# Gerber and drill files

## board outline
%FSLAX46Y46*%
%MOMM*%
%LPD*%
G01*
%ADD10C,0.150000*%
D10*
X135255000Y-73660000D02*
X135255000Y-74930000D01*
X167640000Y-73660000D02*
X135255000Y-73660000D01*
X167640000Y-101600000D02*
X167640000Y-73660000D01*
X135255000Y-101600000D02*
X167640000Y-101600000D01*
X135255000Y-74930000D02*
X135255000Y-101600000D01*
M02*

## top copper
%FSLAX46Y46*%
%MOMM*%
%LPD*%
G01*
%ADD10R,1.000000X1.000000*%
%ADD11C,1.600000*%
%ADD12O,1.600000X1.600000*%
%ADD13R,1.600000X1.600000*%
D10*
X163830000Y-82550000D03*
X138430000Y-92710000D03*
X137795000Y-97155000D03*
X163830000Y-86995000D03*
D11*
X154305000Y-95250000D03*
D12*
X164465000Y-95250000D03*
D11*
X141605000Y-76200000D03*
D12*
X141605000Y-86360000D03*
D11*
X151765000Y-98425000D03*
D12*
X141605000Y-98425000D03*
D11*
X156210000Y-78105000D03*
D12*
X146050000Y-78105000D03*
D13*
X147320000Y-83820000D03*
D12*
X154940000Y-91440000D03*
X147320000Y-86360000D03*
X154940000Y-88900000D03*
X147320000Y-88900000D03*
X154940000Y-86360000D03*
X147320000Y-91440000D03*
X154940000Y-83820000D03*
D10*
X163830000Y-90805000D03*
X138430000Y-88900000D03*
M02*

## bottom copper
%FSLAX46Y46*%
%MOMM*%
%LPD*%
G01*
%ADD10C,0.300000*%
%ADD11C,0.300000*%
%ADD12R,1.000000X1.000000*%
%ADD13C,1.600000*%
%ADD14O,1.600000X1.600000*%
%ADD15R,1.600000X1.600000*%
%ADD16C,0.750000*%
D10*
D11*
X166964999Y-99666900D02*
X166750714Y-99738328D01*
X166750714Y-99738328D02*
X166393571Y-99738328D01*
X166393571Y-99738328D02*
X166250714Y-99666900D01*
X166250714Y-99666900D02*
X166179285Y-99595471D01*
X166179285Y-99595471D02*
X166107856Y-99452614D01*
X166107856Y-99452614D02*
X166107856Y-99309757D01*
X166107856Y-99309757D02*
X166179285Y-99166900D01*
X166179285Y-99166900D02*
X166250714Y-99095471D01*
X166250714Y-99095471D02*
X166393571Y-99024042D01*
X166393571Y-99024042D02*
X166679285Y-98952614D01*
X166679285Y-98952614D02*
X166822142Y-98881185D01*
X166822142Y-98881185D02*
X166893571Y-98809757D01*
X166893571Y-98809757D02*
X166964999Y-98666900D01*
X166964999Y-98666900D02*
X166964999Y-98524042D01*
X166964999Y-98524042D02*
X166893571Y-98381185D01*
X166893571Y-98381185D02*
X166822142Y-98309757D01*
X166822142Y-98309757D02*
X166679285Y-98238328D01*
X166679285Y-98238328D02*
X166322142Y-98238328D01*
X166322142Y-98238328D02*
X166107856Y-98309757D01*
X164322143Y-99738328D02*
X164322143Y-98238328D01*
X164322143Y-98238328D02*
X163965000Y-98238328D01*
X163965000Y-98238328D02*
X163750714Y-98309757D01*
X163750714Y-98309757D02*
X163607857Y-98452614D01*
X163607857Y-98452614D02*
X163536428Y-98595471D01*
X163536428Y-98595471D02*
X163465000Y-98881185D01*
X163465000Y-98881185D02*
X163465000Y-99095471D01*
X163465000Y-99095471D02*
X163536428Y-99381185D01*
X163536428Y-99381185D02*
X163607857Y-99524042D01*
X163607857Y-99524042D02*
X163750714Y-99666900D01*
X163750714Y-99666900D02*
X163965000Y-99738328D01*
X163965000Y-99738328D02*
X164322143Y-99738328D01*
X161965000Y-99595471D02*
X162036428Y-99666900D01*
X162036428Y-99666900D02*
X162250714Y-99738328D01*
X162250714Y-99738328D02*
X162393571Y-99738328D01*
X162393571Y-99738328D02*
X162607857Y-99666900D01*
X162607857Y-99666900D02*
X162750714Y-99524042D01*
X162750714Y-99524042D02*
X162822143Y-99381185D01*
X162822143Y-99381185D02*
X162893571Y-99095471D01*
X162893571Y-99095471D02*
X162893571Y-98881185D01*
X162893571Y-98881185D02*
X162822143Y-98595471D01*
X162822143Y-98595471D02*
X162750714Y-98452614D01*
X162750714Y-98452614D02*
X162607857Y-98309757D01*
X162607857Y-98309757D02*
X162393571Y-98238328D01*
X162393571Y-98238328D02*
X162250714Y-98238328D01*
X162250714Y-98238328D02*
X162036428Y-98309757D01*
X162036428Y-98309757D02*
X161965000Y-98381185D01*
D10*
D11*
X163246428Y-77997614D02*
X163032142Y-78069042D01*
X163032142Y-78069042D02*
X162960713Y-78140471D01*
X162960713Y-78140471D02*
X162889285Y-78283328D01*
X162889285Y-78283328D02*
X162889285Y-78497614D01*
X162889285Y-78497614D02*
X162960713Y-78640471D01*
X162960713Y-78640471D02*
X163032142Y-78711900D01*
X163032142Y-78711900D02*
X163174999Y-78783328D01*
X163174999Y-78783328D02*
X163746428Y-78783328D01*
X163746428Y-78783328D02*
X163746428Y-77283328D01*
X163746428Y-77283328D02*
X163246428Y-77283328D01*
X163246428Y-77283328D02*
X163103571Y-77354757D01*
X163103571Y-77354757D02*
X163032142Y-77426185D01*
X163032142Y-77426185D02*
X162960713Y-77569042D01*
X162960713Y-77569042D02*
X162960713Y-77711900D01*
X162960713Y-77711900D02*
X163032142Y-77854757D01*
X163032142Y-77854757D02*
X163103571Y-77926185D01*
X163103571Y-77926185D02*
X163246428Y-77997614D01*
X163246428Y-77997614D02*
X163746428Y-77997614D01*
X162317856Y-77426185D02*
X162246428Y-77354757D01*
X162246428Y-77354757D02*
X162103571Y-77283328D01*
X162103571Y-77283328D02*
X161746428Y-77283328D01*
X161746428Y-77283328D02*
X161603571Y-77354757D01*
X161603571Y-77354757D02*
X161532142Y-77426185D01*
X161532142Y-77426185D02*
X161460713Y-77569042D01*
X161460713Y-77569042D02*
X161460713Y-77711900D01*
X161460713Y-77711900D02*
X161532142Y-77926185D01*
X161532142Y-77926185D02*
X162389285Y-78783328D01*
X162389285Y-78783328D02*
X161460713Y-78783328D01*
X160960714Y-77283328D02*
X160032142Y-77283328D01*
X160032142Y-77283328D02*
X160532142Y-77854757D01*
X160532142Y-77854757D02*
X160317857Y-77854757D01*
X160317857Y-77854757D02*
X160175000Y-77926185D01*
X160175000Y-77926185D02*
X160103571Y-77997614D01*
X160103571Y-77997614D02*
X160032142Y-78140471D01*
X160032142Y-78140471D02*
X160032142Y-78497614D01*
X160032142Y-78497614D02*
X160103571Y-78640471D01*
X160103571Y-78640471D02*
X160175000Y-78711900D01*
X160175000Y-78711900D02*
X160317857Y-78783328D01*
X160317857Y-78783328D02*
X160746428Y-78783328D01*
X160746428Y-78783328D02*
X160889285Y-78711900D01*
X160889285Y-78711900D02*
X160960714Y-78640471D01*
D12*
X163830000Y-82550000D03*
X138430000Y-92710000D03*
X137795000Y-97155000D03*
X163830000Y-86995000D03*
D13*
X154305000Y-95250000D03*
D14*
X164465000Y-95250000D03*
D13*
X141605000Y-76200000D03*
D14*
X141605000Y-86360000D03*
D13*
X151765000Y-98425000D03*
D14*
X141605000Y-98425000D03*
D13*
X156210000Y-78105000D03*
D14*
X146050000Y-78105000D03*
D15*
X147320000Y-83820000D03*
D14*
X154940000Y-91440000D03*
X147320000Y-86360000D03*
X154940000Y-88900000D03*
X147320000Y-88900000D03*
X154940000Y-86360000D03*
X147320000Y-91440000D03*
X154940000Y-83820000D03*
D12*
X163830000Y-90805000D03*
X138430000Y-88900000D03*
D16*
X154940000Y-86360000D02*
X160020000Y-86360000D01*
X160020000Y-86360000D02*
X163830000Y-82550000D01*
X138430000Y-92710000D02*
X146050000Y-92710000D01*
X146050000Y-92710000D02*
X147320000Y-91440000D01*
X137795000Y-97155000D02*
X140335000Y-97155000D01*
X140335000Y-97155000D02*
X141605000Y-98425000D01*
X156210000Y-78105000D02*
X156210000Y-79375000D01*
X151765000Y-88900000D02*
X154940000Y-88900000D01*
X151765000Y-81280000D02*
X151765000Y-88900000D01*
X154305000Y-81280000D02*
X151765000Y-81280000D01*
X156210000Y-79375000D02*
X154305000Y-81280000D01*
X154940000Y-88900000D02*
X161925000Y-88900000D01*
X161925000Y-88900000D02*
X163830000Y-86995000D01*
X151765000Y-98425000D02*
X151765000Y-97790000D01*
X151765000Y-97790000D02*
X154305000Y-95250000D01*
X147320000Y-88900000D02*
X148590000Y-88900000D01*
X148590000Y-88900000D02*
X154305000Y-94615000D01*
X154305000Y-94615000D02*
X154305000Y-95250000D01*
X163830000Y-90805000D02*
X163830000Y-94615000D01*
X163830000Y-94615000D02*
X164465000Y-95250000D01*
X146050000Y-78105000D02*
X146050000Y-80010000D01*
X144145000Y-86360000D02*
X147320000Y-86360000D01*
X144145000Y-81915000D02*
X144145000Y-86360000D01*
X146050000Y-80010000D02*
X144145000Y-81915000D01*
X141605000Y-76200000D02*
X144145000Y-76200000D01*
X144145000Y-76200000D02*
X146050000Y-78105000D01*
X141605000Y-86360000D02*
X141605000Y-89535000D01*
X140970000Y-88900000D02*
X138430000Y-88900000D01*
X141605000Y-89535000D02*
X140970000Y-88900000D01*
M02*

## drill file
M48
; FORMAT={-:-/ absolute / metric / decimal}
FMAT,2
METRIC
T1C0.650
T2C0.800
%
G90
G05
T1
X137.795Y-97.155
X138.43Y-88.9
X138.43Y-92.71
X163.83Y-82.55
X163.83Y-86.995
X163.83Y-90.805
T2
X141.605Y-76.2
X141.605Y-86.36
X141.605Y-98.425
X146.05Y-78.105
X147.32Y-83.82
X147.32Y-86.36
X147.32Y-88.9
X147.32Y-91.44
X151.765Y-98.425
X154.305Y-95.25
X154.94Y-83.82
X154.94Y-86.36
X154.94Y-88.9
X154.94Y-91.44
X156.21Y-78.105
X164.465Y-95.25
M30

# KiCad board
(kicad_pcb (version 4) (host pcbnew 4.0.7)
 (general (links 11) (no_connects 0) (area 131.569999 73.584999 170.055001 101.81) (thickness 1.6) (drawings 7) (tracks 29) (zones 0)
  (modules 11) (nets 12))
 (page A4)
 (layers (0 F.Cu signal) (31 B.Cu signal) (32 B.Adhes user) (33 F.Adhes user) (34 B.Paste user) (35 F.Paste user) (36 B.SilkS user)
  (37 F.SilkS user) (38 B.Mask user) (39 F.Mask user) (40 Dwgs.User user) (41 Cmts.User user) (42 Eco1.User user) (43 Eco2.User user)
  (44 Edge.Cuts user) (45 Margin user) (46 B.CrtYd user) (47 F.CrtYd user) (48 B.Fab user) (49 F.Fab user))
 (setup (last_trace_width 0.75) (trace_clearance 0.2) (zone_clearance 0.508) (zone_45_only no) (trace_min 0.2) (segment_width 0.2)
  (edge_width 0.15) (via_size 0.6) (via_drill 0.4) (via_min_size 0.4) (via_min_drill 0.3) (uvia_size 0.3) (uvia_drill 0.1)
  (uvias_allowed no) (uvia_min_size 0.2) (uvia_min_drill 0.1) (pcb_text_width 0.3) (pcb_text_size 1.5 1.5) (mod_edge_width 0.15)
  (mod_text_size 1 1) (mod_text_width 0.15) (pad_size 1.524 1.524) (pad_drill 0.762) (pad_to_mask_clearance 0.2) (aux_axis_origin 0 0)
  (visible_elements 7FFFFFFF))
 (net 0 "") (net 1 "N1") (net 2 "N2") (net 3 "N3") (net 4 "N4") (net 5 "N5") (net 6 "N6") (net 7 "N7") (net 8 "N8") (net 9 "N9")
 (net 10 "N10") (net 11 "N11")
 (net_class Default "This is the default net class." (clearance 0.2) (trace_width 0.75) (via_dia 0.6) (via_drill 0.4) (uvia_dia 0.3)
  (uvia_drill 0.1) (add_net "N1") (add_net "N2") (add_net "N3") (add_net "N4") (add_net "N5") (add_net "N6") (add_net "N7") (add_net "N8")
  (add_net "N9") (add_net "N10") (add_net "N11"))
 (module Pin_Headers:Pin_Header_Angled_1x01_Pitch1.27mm (layer F.Cu) (at 163.83 82.55)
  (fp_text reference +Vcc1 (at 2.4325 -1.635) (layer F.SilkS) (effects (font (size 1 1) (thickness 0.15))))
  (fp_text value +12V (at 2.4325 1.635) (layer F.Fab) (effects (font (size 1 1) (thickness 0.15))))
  (pad 1 thru_hole rect (at 0 0) (size 1 1) (drill 0.65) (layers *.Cu *.Mask) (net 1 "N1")))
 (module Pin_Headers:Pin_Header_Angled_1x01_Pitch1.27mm (layer F.Cu) (at 138.43 92.71 180)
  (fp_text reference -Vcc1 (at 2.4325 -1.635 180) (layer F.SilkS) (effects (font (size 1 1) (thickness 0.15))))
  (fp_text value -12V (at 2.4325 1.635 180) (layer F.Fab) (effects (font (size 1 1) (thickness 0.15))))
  (pad 1 thru_hole rect (at 0 0 180) (size 1 1) (drill 0.65) (layers *.Cu *.Mask) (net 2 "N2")))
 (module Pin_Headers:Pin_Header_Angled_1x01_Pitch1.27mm (layer F.Cu) (at 137.795 97.155 180)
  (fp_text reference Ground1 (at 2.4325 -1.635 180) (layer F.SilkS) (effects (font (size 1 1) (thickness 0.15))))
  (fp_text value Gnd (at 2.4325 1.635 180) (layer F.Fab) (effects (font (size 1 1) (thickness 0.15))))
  (pad 1 thru_hole rect (at 0 0 180) (size 1 1) (drill 0.65) (layers *.Cu *.Mask) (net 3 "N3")))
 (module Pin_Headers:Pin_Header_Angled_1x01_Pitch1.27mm (layer F.Cu) (at 163.83 86.995)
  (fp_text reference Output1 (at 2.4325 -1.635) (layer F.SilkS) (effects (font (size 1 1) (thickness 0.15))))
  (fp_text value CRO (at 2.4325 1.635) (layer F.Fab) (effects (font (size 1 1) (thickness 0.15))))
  (pad 1 thru_hole rect (at 0 0) (size 1 1) (drill 0.65) (layers *.Cu *.Mask) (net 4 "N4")))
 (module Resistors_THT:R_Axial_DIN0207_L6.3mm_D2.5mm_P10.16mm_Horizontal (layer F.Cu) (at 154.305 95.25)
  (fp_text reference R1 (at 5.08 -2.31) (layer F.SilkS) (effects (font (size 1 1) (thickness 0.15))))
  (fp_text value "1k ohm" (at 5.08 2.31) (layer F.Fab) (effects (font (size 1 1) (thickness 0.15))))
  (pad 1 thru_hole circle (at 0 0) (size 1.6 1.6) (drill 0.8) (layers *.Cu *.Mask) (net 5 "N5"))
  (pad 2 thru_hole oval (at 10.16 0) (size 1.6 1.6) (drill 0.8) (layers *.Cu *.Mask) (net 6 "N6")))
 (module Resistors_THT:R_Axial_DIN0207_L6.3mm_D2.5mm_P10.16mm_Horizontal (layer F.Cu) (at 141.605 76.2 270)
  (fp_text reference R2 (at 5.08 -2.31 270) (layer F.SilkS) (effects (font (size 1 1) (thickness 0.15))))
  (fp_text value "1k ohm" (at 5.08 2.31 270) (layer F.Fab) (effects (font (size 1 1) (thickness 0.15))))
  (pad 1 thru_hole circle (at 0 0 270) (size 1.6 1.6) (drill 0.8) (layers *.Cu *.Mask) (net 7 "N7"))
  (pad 2 thru_hole oval (at 10.16 0 270) (size 1.6 1.6) (drill 0.8) (layers *.Cu *.Mask) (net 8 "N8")))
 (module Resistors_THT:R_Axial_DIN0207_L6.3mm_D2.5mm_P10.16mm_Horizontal (layer F.Cu) (at 151.765 98.425 180)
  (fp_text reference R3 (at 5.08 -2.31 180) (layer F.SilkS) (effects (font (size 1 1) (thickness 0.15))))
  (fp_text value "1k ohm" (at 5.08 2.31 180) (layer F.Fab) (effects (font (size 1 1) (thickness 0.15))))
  (pad 1 thru_hole circle (at 0 0 180) (size 1.6 1.6) (drill 0.8) (layers *.Cu *.Mask) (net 5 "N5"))
  (pad 2 thru_hole oval (at 10.16 0 180) (size 1.6 1.6) (drill 0.8) (layers *.Cu *.Mask) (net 3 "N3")))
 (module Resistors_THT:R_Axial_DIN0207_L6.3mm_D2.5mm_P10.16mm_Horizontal (layer F.Cu) (at 156.21 78.105 180)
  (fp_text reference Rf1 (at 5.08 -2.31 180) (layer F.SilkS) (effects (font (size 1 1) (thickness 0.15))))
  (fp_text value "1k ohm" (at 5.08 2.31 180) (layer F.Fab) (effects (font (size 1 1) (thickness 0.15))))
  (pad 1 thru_hole circle (at 0 0 180) (size 1.6 1.6) (drill 0.8) (layers *.Cu *.Mask) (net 4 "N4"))
  (pad 2 thru_hole oval (at 10.16 0 180) (size 1.6 1.6) (drill 0.8) (layers *.Cu *.Mask) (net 7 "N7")))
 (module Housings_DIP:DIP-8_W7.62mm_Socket (layer F.Cu) (at 147.32 83.82)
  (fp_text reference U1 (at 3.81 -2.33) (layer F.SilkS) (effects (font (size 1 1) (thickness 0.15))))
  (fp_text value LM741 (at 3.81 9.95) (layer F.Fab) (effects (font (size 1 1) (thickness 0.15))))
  (pad 1 thru_hole rect (at 0 0) (size 1.6 1.6) (drill 0.8) (layers *.Cu *.Mask) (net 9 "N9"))
  (pad 5 thru_hole oval (at 7.62 7.62) (size 1.6 1.6) (drill 0.8) (layers *.Cu *.Mask) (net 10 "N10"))
  (pad 2 thru_hole oval (at 0 2.54) (size 1.6 1.6) (drill 0.8) (layers *.Cu *.Mask) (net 7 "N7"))
  (pad 6 thru_hole oval (at 7.62 5.08) (size 1.6 1.6) (drill 0.8) (layers *.Cu *.Mask) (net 4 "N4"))
  (pad 3 thru_hole oval (at 0 5.08) (size 1.6 1.6) (drill 0.8) (layers *.Cu *.Mask) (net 5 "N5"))
  (pad 7 thru_hole oval (at 7.62 2.54) (size 1.6 1.6) (drill 0.8) (layers *.Cu *.Mask) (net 1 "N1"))
  (pad 4 thru_hole oval (at 0 7.62) (size 1.6 1.6) (drill 0.8) (layers *.Cu *.Mask) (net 2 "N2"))
  (pad 8 thru_hole oval (at 7.62 0) (size 1.6 1.6) (drill 0.8) (layers *.Cu *.Mask) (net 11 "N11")))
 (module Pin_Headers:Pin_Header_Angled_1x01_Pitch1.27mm (layer F.Cu) (at 163.83 90.805)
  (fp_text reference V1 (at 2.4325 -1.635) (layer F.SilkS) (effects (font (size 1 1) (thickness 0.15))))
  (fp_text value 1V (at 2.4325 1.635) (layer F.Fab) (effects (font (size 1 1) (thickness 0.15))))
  (pad 1 thru_hole rect (at 0 0) (size 1 1) (drill 0.65) (layers *.Cu *.Mask) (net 6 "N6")))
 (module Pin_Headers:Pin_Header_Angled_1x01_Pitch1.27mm (layer F.Cu) (at 138.43 88.9 180)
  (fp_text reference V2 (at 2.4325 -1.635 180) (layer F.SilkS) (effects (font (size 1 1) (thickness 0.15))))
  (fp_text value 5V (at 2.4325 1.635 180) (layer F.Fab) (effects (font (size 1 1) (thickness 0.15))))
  (pad 1 thru_hole rect (at 0 0 180) (size 1 1) (drill 0.65) (layers *.Cu *.Mask) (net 8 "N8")))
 (gr_line (start 135.255 73.66) (end 135.255 74.93) (angle 90) (layer Edge.Cuts) (width 0.15))
 (gr_line (start 167.64 73.66) (end 135.255 73.66) (angle 90) (layer Edge.Cuts) (width 0.15))
 (gr_line (start 167.64 101.6) (end 167.64 73.66) (angle 90) (layer Edge.Cuts) (width 0.15))
 (gr_line (start 135.255 101.6) (end 167.64 101.6) (angle 90) (layer Edge.Cuts) (width 0.15))
 (gr_line (start 135.255 74.93) (end 135.255 101.6) (angle 90) (layer Edge.Cuts) (width 0.15))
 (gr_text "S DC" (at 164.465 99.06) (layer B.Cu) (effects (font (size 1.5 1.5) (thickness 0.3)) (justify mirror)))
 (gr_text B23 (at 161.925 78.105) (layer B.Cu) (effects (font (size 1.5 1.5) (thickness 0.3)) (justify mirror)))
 (segment (start 154.94 86.36) (end 160.02 86.36) (width 0.75) (layer B.Cu) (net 1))
 (segment (start 160.02 86.36) (end 163.83 82.55) (width 0.75) (layer B.Cu) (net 1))
 (segment (start 138.43 92.71) (end 146.05 92.71) (width 0.75) (layer B.Cu) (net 2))
 (segment (start 146.05 92.71) (end 147.32 91.44) (width 0.75) (layer B.Cu) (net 2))
 (segment (start 137.795 97.155) (end 140.335 97.155) (width 0.75) (layer B.Cu) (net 3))
 (segment (start 140.335 97.155) (end 141.605 98.425) (width 0.75) (layer B.Cu) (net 3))
 (segment (start 156.21 78.105) (end 156.21 79.375) (width 0.75) (layer B.Cu) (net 4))
 (segment (start 151.765 88.9) (end 154.94 88.9) (width 0.75) (layer B.Cu) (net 4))
 (segment (start 151.765 81.28) (end 151.765 88.9) (width 0.75) (layer B.Cu) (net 4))
 (segment (start 154.305 81.28) (end 151.765 81.28) (width 0.75) (layer B.Cu) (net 4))
 (segment (start 156.21 79.375) (end 154.305 81.28) (width 0.75) (layer B.Cu) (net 4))
 (segment (start 154.94 88.9) (end 161.925 88.9) (width 0.75) (layer B.Cu) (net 4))
 (segment (start 161.925 88.9) (end 163.83 86.995) (width 0.75) (layer B.Cu) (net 4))
 (segment (start 151.765 98.425) (end 151.765 97.79) (width 0.75) (layer B.Cu) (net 5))
 (segment (start 151.765 97.79) (end 154.305 95.25) (width 0.75) (layer B.Cu) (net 5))
 (segment (start 147.32 88.9) (end 148.59 88.9) (width 0.75) (layer B.Cu) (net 5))
 (segment (start 148.59 88.9) (end 154.305 94.615) (width 0.75) (layer B.Cu) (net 5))
 (segment (start 154.305 94.615) (end 154.305 95.25) (width 0.75) (layer B.Cu) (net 5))
 (segment (start 163.83 90.805) (end 163.83 94.615) (width 0.75) (layer B.Cu) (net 6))
 (segment (start 163.83 94.615) (end 164.465 95.25) (width 0.75) (layer B.Cu) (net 6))
 (segment (start 146.05 78.105) (end 146.05 80.01) (width 0.75) (layer B.Cu) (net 7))
 (segment (start 144.145 86.36) (end 147.32 86.36) (width 0.75) (layer B.Cu) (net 7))
 (segment (start 144.145 81.915) (end 144.145 86.36) (width 0.75) (layer B.Cu) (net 7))
 (segment (start 146.05 80.01) (end 144.145 81.915) (width 0.75) (layer B.Cu) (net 7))
 (segment (start 141.605 76.2) (end 144.145 76.2) (width 0.75) (layer B.Cu) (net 7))
 (segment (start 144.145 76.2) (end 146.05 78.105) (width 0.75) (layer B.Cu) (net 7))
 (segment (start 141.605 86.36) (end 141.605 89.535) (width 0.75) (layer B.Cu) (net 8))
 (segment (start 140.97 88.9) (end 138.43 88.9) (width 0.75) (layer B.Cu) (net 8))
 (segment (start 141.605 89.535) (end 140.97 88.9) (width 0.75) (layer B.Cu) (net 8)))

